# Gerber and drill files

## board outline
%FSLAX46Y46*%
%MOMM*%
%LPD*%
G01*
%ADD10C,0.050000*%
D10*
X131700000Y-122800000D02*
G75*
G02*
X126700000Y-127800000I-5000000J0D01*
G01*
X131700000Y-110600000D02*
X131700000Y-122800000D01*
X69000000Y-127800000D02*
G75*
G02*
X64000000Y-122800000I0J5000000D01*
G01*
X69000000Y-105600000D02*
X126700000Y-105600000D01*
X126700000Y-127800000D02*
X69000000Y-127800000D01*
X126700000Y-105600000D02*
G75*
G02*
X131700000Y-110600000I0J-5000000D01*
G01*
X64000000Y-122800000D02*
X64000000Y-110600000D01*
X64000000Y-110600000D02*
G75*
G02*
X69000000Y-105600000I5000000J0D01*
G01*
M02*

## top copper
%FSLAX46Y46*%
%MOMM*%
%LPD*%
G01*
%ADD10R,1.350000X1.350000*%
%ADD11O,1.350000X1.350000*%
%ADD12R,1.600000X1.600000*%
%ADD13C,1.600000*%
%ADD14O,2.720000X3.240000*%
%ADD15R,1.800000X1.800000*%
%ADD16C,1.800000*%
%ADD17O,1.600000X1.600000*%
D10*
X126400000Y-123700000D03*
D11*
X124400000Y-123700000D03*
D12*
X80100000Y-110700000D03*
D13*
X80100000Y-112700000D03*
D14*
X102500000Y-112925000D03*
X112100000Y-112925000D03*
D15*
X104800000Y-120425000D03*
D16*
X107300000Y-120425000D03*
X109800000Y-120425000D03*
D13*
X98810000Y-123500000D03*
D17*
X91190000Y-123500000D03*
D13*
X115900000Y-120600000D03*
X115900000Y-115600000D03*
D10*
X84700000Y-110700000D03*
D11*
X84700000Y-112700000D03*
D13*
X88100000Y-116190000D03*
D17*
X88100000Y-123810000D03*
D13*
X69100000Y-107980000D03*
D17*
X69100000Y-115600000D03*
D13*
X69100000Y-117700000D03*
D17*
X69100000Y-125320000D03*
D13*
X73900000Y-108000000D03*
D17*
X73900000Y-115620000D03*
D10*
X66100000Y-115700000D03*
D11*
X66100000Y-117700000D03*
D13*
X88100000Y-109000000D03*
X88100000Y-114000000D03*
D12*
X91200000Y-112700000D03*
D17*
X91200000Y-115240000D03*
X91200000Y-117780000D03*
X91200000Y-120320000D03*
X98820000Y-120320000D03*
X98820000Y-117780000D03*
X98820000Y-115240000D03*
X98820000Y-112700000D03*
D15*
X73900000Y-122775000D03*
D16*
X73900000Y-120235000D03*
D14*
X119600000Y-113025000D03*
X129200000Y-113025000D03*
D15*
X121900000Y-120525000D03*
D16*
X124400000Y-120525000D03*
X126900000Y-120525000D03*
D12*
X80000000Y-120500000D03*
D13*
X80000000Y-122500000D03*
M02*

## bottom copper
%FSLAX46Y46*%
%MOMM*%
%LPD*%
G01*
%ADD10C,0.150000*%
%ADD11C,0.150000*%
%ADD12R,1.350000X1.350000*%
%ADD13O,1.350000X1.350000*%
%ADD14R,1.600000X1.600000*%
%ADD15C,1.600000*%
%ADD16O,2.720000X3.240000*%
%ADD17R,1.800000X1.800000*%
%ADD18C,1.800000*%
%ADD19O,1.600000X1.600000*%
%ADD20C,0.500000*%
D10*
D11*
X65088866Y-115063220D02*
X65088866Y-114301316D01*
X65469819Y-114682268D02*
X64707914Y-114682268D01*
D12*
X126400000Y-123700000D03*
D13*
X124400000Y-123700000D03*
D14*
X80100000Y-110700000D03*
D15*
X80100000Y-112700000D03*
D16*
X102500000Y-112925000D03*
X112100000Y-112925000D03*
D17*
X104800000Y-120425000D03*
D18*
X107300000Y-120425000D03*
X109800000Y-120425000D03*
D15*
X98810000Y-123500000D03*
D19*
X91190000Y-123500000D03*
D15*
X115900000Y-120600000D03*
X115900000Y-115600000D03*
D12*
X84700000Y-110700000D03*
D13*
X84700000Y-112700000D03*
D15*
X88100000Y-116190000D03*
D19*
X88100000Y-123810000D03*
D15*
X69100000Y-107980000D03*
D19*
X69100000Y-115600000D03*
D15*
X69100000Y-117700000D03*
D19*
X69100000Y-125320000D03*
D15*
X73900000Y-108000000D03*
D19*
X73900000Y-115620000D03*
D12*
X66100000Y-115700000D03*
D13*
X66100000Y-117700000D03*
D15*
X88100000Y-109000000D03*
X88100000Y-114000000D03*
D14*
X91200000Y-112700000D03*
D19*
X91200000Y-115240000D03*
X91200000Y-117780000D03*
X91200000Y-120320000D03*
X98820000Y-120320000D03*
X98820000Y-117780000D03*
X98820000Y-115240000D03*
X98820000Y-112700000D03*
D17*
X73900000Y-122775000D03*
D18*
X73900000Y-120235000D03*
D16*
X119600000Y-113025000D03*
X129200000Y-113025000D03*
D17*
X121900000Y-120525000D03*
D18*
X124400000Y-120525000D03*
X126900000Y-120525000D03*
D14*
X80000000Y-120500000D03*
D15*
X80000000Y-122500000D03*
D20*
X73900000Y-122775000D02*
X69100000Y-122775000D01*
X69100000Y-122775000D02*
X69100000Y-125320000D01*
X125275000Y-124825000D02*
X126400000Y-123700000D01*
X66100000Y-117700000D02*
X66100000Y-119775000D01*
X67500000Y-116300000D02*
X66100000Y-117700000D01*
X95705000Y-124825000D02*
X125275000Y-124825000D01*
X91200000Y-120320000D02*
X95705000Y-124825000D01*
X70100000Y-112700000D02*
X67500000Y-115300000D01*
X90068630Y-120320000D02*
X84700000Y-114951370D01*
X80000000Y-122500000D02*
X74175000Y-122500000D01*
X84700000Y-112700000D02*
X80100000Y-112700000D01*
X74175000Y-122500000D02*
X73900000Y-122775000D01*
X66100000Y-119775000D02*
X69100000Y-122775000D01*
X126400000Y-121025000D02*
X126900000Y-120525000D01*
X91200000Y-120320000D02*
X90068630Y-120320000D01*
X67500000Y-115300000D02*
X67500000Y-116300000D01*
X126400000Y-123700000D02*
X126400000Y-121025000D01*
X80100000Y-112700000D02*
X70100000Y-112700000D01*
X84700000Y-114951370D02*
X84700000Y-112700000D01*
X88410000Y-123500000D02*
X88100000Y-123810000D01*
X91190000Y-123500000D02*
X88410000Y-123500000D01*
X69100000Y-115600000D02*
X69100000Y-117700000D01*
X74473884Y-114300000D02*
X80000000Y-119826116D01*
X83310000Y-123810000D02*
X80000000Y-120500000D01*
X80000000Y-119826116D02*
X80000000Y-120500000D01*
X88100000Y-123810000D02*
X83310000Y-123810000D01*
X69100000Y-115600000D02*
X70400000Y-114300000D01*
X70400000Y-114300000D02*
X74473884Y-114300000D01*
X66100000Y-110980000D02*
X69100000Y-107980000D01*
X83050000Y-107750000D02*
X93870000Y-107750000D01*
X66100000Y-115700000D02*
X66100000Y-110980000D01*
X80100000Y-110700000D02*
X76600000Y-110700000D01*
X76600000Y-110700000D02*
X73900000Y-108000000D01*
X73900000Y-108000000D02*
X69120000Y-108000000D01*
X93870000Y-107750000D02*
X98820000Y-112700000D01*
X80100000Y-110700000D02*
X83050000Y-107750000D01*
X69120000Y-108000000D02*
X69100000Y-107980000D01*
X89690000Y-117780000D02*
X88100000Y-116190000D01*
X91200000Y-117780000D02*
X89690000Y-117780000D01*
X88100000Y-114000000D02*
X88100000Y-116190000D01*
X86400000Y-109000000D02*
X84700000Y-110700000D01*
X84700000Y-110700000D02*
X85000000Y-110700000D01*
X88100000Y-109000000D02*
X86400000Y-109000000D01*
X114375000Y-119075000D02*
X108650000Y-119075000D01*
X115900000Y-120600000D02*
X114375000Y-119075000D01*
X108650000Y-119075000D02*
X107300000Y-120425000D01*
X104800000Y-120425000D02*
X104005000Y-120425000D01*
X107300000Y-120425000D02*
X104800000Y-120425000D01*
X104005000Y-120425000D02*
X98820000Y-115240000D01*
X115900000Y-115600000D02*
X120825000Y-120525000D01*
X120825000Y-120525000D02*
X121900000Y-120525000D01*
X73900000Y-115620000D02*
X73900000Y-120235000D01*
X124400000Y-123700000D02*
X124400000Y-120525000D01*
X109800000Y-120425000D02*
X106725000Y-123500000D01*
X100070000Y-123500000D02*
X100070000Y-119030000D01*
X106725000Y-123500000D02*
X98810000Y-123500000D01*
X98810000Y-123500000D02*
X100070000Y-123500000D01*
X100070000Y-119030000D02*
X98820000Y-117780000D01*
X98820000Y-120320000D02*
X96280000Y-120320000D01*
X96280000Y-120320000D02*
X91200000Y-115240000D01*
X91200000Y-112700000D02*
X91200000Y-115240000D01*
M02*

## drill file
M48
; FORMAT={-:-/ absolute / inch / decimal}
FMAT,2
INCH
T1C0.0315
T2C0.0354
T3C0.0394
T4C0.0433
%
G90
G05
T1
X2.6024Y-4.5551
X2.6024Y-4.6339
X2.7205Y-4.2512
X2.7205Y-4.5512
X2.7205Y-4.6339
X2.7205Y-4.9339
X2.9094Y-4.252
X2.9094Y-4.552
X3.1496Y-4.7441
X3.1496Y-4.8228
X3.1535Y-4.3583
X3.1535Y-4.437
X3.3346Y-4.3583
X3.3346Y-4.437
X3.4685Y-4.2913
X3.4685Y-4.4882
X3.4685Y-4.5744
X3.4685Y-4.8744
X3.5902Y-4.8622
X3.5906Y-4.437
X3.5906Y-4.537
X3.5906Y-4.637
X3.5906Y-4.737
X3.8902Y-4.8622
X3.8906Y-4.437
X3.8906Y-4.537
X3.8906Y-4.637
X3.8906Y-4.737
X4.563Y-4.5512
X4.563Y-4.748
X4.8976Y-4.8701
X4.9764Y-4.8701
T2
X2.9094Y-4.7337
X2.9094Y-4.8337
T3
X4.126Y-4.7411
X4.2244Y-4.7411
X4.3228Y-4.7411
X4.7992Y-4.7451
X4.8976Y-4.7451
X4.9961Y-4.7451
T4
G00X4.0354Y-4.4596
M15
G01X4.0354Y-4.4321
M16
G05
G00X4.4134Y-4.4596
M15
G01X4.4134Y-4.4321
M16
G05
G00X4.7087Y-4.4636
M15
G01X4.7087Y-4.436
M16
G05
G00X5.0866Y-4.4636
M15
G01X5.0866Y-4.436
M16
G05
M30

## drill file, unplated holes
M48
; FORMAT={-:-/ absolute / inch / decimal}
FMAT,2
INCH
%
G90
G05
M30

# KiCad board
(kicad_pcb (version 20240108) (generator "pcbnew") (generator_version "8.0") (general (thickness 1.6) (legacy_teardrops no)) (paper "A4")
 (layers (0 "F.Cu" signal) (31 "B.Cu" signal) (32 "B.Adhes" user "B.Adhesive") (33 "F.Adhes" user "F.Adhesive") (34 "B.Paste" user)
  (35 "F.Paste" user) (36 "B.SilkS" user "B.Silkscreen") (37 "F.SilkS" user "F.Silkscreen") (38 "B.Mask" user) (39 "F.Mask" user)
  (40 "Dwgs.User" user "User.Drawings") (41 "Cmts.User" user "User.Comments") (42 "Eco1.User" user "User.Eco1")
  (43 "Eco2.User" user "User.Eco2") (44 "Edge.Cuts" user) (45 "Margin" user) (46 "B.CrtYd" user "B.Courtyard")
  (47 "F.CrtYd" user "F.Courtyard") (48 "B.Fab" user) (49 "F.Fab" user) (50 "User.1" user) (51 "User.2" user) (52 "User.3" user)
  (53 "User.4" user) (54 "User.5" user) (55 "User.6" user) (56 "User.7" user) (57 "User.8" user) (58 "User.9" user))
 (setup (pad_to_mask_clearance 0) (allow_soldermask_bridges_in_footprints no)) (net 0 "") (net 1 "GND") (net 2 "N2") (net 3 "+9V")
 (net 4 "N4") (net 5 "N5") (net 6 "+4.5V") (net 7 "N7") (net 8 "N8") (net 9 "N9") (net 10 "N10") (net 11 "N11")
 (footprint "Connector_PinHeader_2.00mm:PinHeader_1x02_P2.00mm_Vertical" (layer "F.Cu") (at 126.4 123.7 -90)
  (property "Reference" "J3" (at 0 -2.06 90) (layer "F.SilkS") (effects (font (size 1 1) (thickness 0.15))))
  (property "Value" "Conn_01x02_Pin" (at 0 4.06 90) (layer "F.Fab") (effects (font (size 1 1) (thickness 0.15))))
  (pad "1" thru_hole rect (at 0 0 270) (size 1.35 1.35) (drill 0.8) (layers "*.Cu" "*.Mask") (remove_unused_layers no) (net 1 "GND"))
  (pad "2" thru_hole oval (at 0 2 270) (size 1.35 1.35) (drill 0.8) (layers "*.Cu" "*.Mask") (remove_unused_layers no) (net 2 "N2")))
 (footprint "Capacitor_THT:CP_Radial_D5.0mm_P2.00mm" (layer "F.Cu") (at 80.1 110.7 -90)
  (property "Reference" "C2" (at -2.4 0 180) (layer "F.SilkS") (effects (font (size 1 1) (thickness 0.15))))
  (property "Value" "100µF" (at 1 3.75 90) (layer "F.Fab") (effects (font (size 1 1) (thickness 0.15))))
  (pad "1" thru_hole rect (at 0 0 270) (size 1.6 1.6) (drill 0.8) (layers "*.Cu" "*.Mask") (remove_unused_layers no) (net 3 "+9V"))
  (pad "2" thru_hole circle (at 2 0 270) (size 1.6 1.6) (drill 0.8) (layers "*.Cu" "*.Mask") (remove_unused_layers no) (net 1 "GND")))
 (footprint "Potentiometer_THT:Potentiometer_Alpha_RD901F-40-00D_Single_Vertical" (layer "F.Cu") (at 104.8 120.425 90)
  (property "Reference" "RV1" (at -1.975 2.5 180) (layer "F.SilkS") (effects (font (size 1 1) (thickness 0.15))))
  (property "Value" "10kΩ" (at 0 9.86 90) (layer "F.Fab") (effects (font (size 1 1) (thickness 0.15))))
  (pad "" thru_hole oval (at 7.5 -2.3 180) (size 2.72 3.24) (drill oval 1.1 1.8) (layers "*.Cu" "*.Mask") (remove_unused_layers no))
  (pad "" thru_hole oval (at 7.5 7.3 180) (size 2.72 3.24) (drill oval 1.1 1.8) (layers "*.Cu" "*.Mask") (remove_unused_layers no))
  (pad "1" thru_hole rect (at 0 0 180) (size 1.8 1.8) (drill 1) (layers "*.Cu" "*.Mask") (remove_unused_layers no) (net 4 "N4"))
  (pad "2" thru_hole circle (at 0 2.5 180) (size 1.8 1.8) (drill 1) (layers "*.Cu" "*.Mask") (remove_unused_layers no) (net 4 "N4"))
  (pad "3" thru_hole circle (at 0 5 180) (size 1.8 1.8) (drill 1) (layers "*.Cu" "*.Mask") (remove_unused_layers no) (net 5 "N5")))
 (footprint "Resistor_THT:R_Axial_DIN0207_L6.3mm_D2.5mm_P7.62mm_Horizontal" (layer "F.Cu") (at 98.81 123.5 180)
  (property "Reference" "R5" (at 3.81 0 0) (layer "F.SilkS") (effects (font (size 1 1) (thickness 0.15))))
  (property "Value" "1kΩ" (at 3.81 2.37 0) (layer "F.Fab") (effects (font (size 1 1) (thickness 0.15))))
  (pad "1" thru_hole circle (at 0 0 180) (size 1.6 1.6) (drill 0.8) (layers "*.Cu" "*.Mask") (remove_unused_layers no) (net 5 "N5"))
  (pad "2" thru_hole oval (at 7.62 0 180) (size 1.6 1.6) (drill 0.8) (layers "*.Cu" "*.Mask") (remove_unused_layers no) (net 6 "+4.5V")))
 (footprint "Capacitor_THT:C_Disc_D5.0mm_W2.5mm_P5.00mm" (layer "F.Cu") (at 115.9 120.6 90)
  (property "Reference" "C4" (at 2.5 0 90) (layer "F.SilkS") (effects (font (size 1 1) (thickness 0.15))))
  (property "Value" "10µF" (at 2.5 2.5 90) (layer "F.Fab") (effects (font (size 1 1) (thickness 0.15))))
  (pad "1" thru_hole circle (at 0 0 90) (size 1.6 1.6) (drill 0.8) (layers "*.Cu" "*.Mask") (remove_unused_layers no) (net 4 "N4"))
  (pad "2" thru_hole circle (at 5 0 90) (size 1.6 1.6) (drill 0.8) (layers "*.Cu" "*.Mask") (remove_unused_layers no) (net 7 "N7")))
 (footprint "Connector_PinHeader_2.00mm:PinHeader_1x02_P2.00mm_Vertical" (layer "F.Cu") (at 84.7 110.7)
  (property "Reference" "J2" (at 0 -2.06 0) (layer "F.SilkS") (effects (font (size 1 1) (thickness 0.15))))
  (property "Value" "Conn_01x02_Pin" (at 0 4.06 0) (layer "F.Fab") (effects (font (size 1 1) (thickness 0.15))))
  (pad "1" thru_hole rect (at 0 0) (size 1.35 1.35) (drill 0.8) (layers "*.Cu" "*.Mask") (remove_unused_layers no) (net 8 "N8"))
  (pad "2" thru_hole oval (at 0 2) (size 1.35 1.35) (drill 0.8) (layers "*.Cu" "*.Mask") (remove_unused_layers no) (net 1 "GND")))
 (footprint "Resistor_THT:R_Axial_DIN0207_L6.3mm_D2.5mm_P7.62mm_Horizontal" (layer "F.Cu") (at 88.1 116.19 -90)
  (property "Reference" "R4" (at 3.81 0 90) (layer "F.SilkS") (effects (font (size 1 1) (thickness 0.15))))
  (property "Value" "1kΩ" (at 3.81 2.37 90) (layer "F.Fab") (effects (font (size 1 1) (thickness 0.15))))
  (pad "1" thru_hole circle (at 0 0 270) (size 1.6 1.6) (drill 0.8) (layers "*.Cu" "*.Mask") (remove_unused_layers no) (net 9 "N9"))
  (pad "2" thru_hole oval (at 7.62 0 270) (size 1.6 1.6) (drill 0.8) (layers "*.Cu" "*.Mask") (remove_unused_layers no) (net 6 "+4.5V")))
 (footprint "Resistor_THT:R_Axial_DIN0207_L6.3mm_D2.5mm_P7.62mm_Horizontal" (layer "F.Cu") (at 69.1 107.98 -90)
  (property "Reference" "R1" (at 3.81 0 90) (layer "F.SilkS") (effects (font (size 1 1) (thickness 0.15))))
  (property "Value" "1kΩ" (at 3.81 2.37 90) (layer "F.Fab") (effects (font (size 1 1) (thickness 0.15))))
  (pad "1" thru_hole circle (at 0 0 270) (size 1.6 1.6) (drill 0.8) (layers "*.Cu" "*.Mask") (remove_unused_layers no) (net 3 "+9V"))
  (pad "2" thru_hole oval (at 7.62 0 270) (size 1.6 1.6) (drill 0.8) (layers "*.Cu" "*.Mask") (remove_unused_layers no) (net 6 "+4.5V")))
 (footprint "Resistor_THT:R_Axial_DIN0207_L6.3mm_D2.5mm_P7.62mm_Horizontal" (layer "F.Cu") (at 69.1 117.7 -90)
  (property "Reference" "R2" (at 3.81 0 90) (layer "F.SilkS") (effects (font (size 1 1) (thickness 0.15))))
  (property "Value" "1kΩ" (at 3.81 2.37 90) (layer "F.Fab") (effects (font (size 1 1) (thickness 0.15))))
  (pad "1" thru_hole circle (at 0 0 270) (size 1.6 1.6) (drill 0.8) (layers "*.Cu" "*.Mask") (remove_unused_layers no) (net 6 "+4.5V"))
  (pad "2" thru_hole oval (at 7.62 0 270) (size 1.6 1.6) (drill 0.8) (layers "*.Cu" "*.Mask") (remove_unused_layers no) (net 1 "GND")))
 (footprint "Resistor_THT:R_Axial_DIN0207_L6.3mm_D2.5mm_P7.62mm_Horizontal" (layer "F.Cu") (at 73.9 108 -90)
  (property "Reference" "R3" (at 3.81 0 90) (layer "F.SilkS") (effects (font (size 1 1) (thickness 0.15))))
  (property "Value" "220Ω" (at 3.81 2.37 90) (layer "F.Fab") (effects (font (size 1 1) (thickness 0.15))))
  (pad "1" thru_hole circle (at 0 0 270) (size 1.6 1.6) (drill 0.8) (layers "*.Cu" "*.Mask") (remove_unused_layers no) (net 3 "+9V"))
  (pad "2" thru_hole oval (at 7.62 0 270) (size 1.6 1.6) (drill 0.8) (layers "*.Cu" "*.Mask") (remove_unused_layers no) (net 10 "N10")))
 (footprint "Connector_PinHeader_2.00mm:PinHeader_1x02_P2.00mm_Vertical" (layer "F.Cu") (at 66.1 115.7)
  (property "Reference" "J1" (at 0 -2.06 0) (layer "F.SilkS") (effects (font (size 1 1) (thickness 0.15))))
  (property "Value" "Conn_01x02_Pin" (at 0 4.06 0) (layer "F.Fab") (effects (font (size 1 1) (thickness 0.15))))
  (pad "1" thru_hole rect (at 0 0) (size 1.35 1.35) (drill 0.8) (layers "*.Cu" "*.Mask") (remove_unused_layers no) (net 3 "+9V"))
  (pad "2" thru_hole oval (at 0 2) (size 1.35 1.35) (drill 0.8) (layers "*.Cu" "*.Mask") (remove_unused_layers no) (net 1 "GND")))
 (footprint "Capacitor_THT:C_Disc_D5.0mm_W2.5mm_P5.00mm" (layer "F.Cu") (at 88.1 109 -90)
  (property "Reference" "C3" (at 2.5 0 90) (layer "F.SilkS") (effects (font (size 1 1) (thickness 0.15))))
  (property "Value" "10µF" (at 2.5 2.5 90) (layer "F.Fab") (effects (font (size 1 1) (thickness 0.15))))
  (pad "1" thru_hole circle (at 0 0 270) (size 1.6 1.6) (drill 0.8) (layers "*.Cu" "*.Mask") (remove_unused_layers no) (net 8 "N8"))
  (pad "2" thru_hole circle (at 5 0 270) (size 1.6 1.6) (drill 0.8) (layers "*.Cu" "*.Mask") (remove_unused_layers no) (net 9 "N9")))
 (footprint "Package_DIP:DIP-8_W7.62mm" (layer "F.Cu") (at 91.2 112.7)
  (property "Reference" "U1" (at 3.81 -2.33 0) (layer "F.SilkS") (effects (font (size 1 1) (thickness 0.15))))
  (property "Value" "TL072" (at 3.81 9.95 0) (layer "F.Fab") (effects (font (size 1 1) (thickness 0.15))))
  (pad "1" thru_hole rect (at 0 0) (size 1.6 1.6) (drill 0.8) (layers "*.Cu" "*.Mask") (remove_unused_layers no) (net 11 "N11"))
  (pad "2" thru_hole oval (at 0 2.54) (size 1.6 1.6) (drill 0.8) (layers "*.Cu" "*.Mask") (remove_unused_layers no) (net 11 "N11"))
  (pad "3" thru_hole oval (at 0 5.08) (size 1.6 1.6) (drill 0.8) (layers "*.Cu" "*.Mask") (remove_unused_layers no) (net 9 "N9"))
  (pad "4" thru_hole oval (at 0 7.62) (size 1.6 1.6) (drill 0.8) (layers "*.Cu" "*.Mask") (remove_unused_layers no) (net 1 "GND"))
  (pad "5" thru_hole oval (at 7.62 7.62) (size 1.6 1.6) (drill 0.8) (layers "*.Cu" "*.Mask") (remove_unused_layers no) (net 11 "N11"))
  (pad "6" thru_hole oval (at 7.62 5.08) (size 1.6 1.6) (drill 0.8) (layers "*.Cu" "*.Mask") (remove_unused_layers no) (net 5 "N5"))
  (pad "7" thru_hole oval (at 7.62 2.54) (size 1.6 1.6) (drill 0.8) (layers "*.Cu" "*.Mask") (remove_unused_layers no) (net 4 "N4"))
  (pad "8" thru_hole oval (at 7.62 0) (size 1.6 1.6) (drill 0.8) (layers "*.Cu" "*.Mask") (remove_unused_layers no) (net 3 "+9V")))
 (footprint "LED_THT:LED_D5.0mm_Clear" (layer "F.Cu") (at 73.9 122.775 90)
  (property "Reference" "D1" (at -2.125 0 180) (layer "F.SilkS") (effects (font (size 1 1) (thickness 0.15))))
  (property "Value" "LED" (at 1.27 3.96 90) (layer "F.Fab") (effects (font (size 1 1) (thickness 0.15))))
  (pad "1" thru_hole rect (at 0 0 90) (size 1.8 1.8) (drill 0.9) (layers "*.Cu" "*.Mask") (remove_unused_layers no) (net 1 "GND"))
  (pad "2" thru_hole circle (at 2.54 0 90) (size 1.8 1.8) (drill 0.9) (layers "*.Cu" "*.Mask") (remove_unused_layers no) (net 10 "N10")))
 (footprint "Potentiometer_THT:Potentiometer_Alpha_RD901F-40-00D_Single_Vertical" (layer "F.Cu") (at 121.9 120.525 90)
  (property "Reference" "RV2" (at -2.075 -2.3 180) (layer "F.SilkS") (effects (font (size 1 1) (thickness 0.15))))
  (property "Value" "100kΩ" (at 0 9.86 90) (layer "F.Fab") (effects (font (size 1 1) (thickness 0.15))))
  (pad "" thru_hole oval (at 7.5 -2.3 180) (size 2.72 3.24) (drill oval 1.1 1.8) (layers "*.Cu" "*.Mask") (remove_unused_layers no))
  (pad "" thru_hole oval (at 7.5 7.3 180) (size 2.72 3.24) (drill oval 1.1 1.8) (layers "*.Cu" "*.Mask") (remove_unused_layers no))
  (pad "1" thru_hole rect (at 0 0 180) (size 1.8 1.8) (drill 1) (layers "*.Cu" "*.Mask") (remove_unused_layers no) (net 7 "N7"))
  (pad "2" thru_hole circle (at 0 2.5 180) (size 1.8 1.8) (drill 1) (layers "*.Cu" "*.Mask") (remove_unused_layers no) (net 2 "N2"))
  (pad "3" thru_hole circle (at 0 5 180) (size 1.8 1.8) (drill 1) (layers "*.Cu" "*.Mask") (remove_unused_layers no) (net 1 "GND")))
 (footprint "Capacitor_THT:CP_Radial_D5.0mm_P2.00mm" (layer "F.Cu") (at 80 120.5 -90)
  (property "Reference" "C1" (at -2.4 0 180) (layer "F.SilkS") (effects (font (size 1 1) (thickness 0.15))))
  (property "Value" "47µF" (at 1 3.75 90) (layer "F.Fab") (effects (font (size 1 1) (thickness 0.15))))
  (pad "1" thru_hole rect (at 0 0 270) (size 1.6 1.6) (drill 0.8) (layers "*.Cu" "*.Mask") (remove_unused_layers no) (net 6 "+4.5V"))
  (pad "2" thru_hole circle (at 2 0 270) (size 1.6 1.6) (drill 0.8) (layers "*.Cu" "*.Mask") (remove_unused_layers no) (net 1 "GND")))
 (gr_arc (start 131.7 122.8) (mid 130.235534 126.335534) (end 126.7 127.8) (stroke (width 0.05) (type default)) (layer "Edge.Cuts"))
 (gr_line (start 131.7 110.6) (end 131.7 122.8) (stroke (width 0.05) (type default)) (layer "Edge.Cuts"))
 (gr_arc (start 69 127.8) (mid 65.464466 126.335534) (end 64 122.8) (stroke (width 0.05) (type default)) (layer "Edge.Cuts"))
 (gr_line (start 69 105.6) (end 126.7 105.6) (stroke (width 0.05) (type default)) (layer "Edge.Cuts"))
 (gr_line (start 126.7 127.8) (end 69 127.8) (stroke (width 0.05) (type default)) (layer "Edge.Cuts"))
 (gr_arc (start 126.7 105.6) (mid 130.235534 107.064466) (end 131.7 110.6) (stroke (width 0.05) (type default)) (layer "Edge.Cuts"))
 (gr_line (start 64 122.8) (end 64 110.6) (stroke (width 0.05) (type default)) (layer "Edge.Cuts"))
 (gr_arc (start 64 110.6) (mid 65.464466 107.064466) (end 69 105.6) (stroke (width 0.05) (type default)) (layer "Edge.Cuts"))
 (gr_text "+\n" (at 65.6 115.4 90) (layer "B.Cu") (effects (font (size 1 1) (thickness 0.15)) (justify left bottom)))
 (segment (start 73.9 122.775) (end 69.1 122.775) (width 0.5) (layer "B.Cu") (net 1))
 (segment (start 69.1 122.775) (end 69.1 125.32) (width 0.5) (layer "B.Cu") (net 1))
 (segment (start 125.275 124.825) (end 126.4 123.7) (width 0.5) (layer "B.Cu") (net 1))
 (segment (start 66.1 117.7) (end 66.1 119.775) (width 0.5) (layer "B.Cu") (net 1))
 (segment (start 67.5 116.3) (end 66.1 117.7) (width 0.5) (layer "B.Cu") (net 1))
 (segment (start 95.705 124.825) (end 125.275 124.825) (width 0.5) (layer "B.Cu") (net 1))
 (segment (start 91.2 120.32) (end 95.705 124.825) (width 0.5) (layer "B.Cu") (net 1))
 (segment (start 70.1 112.7) (end 67.5 115.3) (width 0.5) (layer "B.Cu") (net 1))
 (segment (start 90.06863 120.32) (end 84.7 114.95137) (width 0.5) (layer "B.Cu") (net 1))
 (segment (start 80 122.5) (end 74.175 122.5) (width 0.5) (layer "B.Cu") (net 1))
 (segment (start 84.7 112.7) (end 80.1 112.7) (width 0.5) (layer "B.Cu") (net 1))
 (segment (start 74.175 122.5) (end 73.9 122.775) (width 0.5) (layer "B.Cu") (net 1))
 (segment (start 66.1 119.775) (end 69.1 122.775) (width 0.5) (layer "B.Cu") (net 1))
 (segment (start 126.4 121.025) (end 126.9 120.525) (width 0.5) (layer "B.Cu") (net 1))
 (segment (start 91.2 120.32) (end 90.06863 120.32) (width 0.5) (layer "B.Cu") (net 1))
 (segment (start 67.5 115.3) (end 67.5 116.3) (width 0.5) (layer "B.Cu") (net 1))
 (segment (start 126.4 123.7) (end 126.4 121.025) (width 0.5) (layer "B.Cu") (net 1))
 (segment (start 80.1 112.7) (end 70.1 112.7) (width 0.5) (layer "B.Cu") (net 1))
 (segment (start 84.7 114.95137) (end 84.7 112.7) (width 0.5) (layer "B.Cu") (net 1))
 (segment (start 88.41 123.5) (end 88.1 123.81) (width 0.5) (layer "B.Cu") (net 6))
 (segment (start 91.19 123.5) (end 88.41 123.5) (width 0.5) (layer "B.Cu") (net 6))
 (segment (start 69.1 115.6) (end 69.1 117.7) (width 0.5) (layer "B.Cu") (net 6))
 (segment (start 74.473884 114.3) (end 80 119.826116) (width 0.5) (layer "B.Cu") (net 6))
 (segment (start 83.31 123.81) (end 80 120.5) (width 0.5) (layer "B.Cu") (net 6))
 (segment (start 80 119.826116) (end 80 120.5) (width 0.5) (layer "B.Cu") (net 6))
 (segment (start 88.1 123.81) (end 83.31 123.81) (width 0.5) (layer "B.Cu") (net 6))
 (segment (start 69.1 115.6) (end 70.4 114.3) (width 0.5) (layer "B.Cu") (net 6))
 (segment (start 70.4 114.3) (end 74.473884 114.3) (width 0.5) (layer "B.Cu") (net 6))
 (segment (start 66.1 110.98) (end 69.1 107.98) (width 0.5) (layer "B.Cu") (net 3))
 (segment (start 83.05 107.75) (end 93.87 107.75) (width 0.5) (layer "B.Cu") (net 3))
 (segment (start 66.1 115.7) (end 66.1 110.98) (width 0.5) (layer "B.Cu") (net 3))
 (segment (start 80.1 110.7) (end 76.6 110.7) (width 0.5) (layer "B.Cu") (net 3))
 (segment (start 76.6 110.7) (end 73.9 108) (width 0.5) (layer "B.Cu") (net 3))
 (segment (start 73.9 108) (end 69.12 108) (width 0.5) (layer "B.Cu") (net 3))
 (segment (start 93.87 107.75) (end 98.82 112.7) (width 0.5) (layer "B.Cu") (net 3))
 (segment (start 80.1 110.7) (end 83.05 107.75) (width 0.5) (layer "B.Cu") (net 3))
 (segment (start 69.12 108) (end 69.1 107.98) (width 0.5) (layer "B.Cu") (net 3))
 (segment (start 89.69 117.78) (end 88.1 116.19) (width 0.5) (layer "B.Cu") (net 9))
 (segment (start 91.2 117.78) (end 89.69 117.78) (width 0.5) (layer "B.Cu") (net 9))
 (segment (start 88.1 114) (end 88.1 116.19) (width 0.5) (layer "B.Cu") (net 9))
 (segment (start 86.4 109) (end 84.7 110.7) (width 0.5) (layer "B.Cu") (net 8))
 (segment (start 84.7 110.7) (end 85 110.7) (width 0.5) (layer "B.Cu") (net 8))
 (segment (start 88.1 109) (end 86.4 109) (width 0.5) (layer "B.Cu") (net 8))
 (segment (start 114.375 119.075) (end 108.65 119.075) (width 0.5) (layer "B.Cu") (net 4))
 (segment (start 115.9 120.6) (end 114.375 119.075) (width 0.5) (layer "B.Cu") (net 4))
 (segment (start 108.65 119.075) (end 107.3 120.425) (width 0.5) (layer "B.Cu") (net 4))
 (segment (start 104.8 120.425) (end 104.005 120.425) (width 0.5) (layer "B.Cu") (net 4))
 (segment (start 107.3 120.425) (end 104.8 120.425) (width 0.5) (layer "B.Cu") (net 4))
 (segment (start 104.005 120.425) (end 98.82 115.24) (width 0.5) (layer "B.Cu") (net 4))
 (segment (start 115.9 115.6) (end 120.825 120.525) (width 0.5) (layer "B.Cu") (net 7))
 (segment (start 120.825 120.525) (end 121.9 120.525) (width 0.5) (layer "B.Cu") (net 7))
 (segment (start 73.9 115.62) (end 73.9 120.235) (width 0.5) (layer "B.Cu") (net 10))
 (segment (start 124.4 123.7) (end 124.4 120.525) (width 0.5) (layer "B.Cu") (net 2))
 (segment (start 109.8 120.425) (end 106.725 123.5) (width 0.5) (layer "B.Cu") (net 5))
 (segment (start 100.07 123.5) (end 100.07 119.03) (width 0.5) (layer "B.Cu") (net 5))
 (segment (start 106.725 123.5) (end 98.81 123.5) (width 0.5) (layer "B.Cu") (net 5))
 (segment (start 98.81 123.5) (end 100.07 123.5) (width 0.5) (layer "B.Cu") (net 5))
 (segment (start 100.07 119.03) (end 98.82 117.78) (width 0.5) (layer "B.Cu") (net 5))
 (segment (start 98.82 120.32) (end 96.28 120.32) (width 0.5) (layer "B.Cu") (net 11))
 (segment (start 96.28 120.32) (end 91.2 115.24) (width 0.5) (layer "B.Cu") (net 11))
 (segment (start 91.2 112.7) (end 91.2 115.24) (width 0.5) (layer "B.Cu") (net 11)))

